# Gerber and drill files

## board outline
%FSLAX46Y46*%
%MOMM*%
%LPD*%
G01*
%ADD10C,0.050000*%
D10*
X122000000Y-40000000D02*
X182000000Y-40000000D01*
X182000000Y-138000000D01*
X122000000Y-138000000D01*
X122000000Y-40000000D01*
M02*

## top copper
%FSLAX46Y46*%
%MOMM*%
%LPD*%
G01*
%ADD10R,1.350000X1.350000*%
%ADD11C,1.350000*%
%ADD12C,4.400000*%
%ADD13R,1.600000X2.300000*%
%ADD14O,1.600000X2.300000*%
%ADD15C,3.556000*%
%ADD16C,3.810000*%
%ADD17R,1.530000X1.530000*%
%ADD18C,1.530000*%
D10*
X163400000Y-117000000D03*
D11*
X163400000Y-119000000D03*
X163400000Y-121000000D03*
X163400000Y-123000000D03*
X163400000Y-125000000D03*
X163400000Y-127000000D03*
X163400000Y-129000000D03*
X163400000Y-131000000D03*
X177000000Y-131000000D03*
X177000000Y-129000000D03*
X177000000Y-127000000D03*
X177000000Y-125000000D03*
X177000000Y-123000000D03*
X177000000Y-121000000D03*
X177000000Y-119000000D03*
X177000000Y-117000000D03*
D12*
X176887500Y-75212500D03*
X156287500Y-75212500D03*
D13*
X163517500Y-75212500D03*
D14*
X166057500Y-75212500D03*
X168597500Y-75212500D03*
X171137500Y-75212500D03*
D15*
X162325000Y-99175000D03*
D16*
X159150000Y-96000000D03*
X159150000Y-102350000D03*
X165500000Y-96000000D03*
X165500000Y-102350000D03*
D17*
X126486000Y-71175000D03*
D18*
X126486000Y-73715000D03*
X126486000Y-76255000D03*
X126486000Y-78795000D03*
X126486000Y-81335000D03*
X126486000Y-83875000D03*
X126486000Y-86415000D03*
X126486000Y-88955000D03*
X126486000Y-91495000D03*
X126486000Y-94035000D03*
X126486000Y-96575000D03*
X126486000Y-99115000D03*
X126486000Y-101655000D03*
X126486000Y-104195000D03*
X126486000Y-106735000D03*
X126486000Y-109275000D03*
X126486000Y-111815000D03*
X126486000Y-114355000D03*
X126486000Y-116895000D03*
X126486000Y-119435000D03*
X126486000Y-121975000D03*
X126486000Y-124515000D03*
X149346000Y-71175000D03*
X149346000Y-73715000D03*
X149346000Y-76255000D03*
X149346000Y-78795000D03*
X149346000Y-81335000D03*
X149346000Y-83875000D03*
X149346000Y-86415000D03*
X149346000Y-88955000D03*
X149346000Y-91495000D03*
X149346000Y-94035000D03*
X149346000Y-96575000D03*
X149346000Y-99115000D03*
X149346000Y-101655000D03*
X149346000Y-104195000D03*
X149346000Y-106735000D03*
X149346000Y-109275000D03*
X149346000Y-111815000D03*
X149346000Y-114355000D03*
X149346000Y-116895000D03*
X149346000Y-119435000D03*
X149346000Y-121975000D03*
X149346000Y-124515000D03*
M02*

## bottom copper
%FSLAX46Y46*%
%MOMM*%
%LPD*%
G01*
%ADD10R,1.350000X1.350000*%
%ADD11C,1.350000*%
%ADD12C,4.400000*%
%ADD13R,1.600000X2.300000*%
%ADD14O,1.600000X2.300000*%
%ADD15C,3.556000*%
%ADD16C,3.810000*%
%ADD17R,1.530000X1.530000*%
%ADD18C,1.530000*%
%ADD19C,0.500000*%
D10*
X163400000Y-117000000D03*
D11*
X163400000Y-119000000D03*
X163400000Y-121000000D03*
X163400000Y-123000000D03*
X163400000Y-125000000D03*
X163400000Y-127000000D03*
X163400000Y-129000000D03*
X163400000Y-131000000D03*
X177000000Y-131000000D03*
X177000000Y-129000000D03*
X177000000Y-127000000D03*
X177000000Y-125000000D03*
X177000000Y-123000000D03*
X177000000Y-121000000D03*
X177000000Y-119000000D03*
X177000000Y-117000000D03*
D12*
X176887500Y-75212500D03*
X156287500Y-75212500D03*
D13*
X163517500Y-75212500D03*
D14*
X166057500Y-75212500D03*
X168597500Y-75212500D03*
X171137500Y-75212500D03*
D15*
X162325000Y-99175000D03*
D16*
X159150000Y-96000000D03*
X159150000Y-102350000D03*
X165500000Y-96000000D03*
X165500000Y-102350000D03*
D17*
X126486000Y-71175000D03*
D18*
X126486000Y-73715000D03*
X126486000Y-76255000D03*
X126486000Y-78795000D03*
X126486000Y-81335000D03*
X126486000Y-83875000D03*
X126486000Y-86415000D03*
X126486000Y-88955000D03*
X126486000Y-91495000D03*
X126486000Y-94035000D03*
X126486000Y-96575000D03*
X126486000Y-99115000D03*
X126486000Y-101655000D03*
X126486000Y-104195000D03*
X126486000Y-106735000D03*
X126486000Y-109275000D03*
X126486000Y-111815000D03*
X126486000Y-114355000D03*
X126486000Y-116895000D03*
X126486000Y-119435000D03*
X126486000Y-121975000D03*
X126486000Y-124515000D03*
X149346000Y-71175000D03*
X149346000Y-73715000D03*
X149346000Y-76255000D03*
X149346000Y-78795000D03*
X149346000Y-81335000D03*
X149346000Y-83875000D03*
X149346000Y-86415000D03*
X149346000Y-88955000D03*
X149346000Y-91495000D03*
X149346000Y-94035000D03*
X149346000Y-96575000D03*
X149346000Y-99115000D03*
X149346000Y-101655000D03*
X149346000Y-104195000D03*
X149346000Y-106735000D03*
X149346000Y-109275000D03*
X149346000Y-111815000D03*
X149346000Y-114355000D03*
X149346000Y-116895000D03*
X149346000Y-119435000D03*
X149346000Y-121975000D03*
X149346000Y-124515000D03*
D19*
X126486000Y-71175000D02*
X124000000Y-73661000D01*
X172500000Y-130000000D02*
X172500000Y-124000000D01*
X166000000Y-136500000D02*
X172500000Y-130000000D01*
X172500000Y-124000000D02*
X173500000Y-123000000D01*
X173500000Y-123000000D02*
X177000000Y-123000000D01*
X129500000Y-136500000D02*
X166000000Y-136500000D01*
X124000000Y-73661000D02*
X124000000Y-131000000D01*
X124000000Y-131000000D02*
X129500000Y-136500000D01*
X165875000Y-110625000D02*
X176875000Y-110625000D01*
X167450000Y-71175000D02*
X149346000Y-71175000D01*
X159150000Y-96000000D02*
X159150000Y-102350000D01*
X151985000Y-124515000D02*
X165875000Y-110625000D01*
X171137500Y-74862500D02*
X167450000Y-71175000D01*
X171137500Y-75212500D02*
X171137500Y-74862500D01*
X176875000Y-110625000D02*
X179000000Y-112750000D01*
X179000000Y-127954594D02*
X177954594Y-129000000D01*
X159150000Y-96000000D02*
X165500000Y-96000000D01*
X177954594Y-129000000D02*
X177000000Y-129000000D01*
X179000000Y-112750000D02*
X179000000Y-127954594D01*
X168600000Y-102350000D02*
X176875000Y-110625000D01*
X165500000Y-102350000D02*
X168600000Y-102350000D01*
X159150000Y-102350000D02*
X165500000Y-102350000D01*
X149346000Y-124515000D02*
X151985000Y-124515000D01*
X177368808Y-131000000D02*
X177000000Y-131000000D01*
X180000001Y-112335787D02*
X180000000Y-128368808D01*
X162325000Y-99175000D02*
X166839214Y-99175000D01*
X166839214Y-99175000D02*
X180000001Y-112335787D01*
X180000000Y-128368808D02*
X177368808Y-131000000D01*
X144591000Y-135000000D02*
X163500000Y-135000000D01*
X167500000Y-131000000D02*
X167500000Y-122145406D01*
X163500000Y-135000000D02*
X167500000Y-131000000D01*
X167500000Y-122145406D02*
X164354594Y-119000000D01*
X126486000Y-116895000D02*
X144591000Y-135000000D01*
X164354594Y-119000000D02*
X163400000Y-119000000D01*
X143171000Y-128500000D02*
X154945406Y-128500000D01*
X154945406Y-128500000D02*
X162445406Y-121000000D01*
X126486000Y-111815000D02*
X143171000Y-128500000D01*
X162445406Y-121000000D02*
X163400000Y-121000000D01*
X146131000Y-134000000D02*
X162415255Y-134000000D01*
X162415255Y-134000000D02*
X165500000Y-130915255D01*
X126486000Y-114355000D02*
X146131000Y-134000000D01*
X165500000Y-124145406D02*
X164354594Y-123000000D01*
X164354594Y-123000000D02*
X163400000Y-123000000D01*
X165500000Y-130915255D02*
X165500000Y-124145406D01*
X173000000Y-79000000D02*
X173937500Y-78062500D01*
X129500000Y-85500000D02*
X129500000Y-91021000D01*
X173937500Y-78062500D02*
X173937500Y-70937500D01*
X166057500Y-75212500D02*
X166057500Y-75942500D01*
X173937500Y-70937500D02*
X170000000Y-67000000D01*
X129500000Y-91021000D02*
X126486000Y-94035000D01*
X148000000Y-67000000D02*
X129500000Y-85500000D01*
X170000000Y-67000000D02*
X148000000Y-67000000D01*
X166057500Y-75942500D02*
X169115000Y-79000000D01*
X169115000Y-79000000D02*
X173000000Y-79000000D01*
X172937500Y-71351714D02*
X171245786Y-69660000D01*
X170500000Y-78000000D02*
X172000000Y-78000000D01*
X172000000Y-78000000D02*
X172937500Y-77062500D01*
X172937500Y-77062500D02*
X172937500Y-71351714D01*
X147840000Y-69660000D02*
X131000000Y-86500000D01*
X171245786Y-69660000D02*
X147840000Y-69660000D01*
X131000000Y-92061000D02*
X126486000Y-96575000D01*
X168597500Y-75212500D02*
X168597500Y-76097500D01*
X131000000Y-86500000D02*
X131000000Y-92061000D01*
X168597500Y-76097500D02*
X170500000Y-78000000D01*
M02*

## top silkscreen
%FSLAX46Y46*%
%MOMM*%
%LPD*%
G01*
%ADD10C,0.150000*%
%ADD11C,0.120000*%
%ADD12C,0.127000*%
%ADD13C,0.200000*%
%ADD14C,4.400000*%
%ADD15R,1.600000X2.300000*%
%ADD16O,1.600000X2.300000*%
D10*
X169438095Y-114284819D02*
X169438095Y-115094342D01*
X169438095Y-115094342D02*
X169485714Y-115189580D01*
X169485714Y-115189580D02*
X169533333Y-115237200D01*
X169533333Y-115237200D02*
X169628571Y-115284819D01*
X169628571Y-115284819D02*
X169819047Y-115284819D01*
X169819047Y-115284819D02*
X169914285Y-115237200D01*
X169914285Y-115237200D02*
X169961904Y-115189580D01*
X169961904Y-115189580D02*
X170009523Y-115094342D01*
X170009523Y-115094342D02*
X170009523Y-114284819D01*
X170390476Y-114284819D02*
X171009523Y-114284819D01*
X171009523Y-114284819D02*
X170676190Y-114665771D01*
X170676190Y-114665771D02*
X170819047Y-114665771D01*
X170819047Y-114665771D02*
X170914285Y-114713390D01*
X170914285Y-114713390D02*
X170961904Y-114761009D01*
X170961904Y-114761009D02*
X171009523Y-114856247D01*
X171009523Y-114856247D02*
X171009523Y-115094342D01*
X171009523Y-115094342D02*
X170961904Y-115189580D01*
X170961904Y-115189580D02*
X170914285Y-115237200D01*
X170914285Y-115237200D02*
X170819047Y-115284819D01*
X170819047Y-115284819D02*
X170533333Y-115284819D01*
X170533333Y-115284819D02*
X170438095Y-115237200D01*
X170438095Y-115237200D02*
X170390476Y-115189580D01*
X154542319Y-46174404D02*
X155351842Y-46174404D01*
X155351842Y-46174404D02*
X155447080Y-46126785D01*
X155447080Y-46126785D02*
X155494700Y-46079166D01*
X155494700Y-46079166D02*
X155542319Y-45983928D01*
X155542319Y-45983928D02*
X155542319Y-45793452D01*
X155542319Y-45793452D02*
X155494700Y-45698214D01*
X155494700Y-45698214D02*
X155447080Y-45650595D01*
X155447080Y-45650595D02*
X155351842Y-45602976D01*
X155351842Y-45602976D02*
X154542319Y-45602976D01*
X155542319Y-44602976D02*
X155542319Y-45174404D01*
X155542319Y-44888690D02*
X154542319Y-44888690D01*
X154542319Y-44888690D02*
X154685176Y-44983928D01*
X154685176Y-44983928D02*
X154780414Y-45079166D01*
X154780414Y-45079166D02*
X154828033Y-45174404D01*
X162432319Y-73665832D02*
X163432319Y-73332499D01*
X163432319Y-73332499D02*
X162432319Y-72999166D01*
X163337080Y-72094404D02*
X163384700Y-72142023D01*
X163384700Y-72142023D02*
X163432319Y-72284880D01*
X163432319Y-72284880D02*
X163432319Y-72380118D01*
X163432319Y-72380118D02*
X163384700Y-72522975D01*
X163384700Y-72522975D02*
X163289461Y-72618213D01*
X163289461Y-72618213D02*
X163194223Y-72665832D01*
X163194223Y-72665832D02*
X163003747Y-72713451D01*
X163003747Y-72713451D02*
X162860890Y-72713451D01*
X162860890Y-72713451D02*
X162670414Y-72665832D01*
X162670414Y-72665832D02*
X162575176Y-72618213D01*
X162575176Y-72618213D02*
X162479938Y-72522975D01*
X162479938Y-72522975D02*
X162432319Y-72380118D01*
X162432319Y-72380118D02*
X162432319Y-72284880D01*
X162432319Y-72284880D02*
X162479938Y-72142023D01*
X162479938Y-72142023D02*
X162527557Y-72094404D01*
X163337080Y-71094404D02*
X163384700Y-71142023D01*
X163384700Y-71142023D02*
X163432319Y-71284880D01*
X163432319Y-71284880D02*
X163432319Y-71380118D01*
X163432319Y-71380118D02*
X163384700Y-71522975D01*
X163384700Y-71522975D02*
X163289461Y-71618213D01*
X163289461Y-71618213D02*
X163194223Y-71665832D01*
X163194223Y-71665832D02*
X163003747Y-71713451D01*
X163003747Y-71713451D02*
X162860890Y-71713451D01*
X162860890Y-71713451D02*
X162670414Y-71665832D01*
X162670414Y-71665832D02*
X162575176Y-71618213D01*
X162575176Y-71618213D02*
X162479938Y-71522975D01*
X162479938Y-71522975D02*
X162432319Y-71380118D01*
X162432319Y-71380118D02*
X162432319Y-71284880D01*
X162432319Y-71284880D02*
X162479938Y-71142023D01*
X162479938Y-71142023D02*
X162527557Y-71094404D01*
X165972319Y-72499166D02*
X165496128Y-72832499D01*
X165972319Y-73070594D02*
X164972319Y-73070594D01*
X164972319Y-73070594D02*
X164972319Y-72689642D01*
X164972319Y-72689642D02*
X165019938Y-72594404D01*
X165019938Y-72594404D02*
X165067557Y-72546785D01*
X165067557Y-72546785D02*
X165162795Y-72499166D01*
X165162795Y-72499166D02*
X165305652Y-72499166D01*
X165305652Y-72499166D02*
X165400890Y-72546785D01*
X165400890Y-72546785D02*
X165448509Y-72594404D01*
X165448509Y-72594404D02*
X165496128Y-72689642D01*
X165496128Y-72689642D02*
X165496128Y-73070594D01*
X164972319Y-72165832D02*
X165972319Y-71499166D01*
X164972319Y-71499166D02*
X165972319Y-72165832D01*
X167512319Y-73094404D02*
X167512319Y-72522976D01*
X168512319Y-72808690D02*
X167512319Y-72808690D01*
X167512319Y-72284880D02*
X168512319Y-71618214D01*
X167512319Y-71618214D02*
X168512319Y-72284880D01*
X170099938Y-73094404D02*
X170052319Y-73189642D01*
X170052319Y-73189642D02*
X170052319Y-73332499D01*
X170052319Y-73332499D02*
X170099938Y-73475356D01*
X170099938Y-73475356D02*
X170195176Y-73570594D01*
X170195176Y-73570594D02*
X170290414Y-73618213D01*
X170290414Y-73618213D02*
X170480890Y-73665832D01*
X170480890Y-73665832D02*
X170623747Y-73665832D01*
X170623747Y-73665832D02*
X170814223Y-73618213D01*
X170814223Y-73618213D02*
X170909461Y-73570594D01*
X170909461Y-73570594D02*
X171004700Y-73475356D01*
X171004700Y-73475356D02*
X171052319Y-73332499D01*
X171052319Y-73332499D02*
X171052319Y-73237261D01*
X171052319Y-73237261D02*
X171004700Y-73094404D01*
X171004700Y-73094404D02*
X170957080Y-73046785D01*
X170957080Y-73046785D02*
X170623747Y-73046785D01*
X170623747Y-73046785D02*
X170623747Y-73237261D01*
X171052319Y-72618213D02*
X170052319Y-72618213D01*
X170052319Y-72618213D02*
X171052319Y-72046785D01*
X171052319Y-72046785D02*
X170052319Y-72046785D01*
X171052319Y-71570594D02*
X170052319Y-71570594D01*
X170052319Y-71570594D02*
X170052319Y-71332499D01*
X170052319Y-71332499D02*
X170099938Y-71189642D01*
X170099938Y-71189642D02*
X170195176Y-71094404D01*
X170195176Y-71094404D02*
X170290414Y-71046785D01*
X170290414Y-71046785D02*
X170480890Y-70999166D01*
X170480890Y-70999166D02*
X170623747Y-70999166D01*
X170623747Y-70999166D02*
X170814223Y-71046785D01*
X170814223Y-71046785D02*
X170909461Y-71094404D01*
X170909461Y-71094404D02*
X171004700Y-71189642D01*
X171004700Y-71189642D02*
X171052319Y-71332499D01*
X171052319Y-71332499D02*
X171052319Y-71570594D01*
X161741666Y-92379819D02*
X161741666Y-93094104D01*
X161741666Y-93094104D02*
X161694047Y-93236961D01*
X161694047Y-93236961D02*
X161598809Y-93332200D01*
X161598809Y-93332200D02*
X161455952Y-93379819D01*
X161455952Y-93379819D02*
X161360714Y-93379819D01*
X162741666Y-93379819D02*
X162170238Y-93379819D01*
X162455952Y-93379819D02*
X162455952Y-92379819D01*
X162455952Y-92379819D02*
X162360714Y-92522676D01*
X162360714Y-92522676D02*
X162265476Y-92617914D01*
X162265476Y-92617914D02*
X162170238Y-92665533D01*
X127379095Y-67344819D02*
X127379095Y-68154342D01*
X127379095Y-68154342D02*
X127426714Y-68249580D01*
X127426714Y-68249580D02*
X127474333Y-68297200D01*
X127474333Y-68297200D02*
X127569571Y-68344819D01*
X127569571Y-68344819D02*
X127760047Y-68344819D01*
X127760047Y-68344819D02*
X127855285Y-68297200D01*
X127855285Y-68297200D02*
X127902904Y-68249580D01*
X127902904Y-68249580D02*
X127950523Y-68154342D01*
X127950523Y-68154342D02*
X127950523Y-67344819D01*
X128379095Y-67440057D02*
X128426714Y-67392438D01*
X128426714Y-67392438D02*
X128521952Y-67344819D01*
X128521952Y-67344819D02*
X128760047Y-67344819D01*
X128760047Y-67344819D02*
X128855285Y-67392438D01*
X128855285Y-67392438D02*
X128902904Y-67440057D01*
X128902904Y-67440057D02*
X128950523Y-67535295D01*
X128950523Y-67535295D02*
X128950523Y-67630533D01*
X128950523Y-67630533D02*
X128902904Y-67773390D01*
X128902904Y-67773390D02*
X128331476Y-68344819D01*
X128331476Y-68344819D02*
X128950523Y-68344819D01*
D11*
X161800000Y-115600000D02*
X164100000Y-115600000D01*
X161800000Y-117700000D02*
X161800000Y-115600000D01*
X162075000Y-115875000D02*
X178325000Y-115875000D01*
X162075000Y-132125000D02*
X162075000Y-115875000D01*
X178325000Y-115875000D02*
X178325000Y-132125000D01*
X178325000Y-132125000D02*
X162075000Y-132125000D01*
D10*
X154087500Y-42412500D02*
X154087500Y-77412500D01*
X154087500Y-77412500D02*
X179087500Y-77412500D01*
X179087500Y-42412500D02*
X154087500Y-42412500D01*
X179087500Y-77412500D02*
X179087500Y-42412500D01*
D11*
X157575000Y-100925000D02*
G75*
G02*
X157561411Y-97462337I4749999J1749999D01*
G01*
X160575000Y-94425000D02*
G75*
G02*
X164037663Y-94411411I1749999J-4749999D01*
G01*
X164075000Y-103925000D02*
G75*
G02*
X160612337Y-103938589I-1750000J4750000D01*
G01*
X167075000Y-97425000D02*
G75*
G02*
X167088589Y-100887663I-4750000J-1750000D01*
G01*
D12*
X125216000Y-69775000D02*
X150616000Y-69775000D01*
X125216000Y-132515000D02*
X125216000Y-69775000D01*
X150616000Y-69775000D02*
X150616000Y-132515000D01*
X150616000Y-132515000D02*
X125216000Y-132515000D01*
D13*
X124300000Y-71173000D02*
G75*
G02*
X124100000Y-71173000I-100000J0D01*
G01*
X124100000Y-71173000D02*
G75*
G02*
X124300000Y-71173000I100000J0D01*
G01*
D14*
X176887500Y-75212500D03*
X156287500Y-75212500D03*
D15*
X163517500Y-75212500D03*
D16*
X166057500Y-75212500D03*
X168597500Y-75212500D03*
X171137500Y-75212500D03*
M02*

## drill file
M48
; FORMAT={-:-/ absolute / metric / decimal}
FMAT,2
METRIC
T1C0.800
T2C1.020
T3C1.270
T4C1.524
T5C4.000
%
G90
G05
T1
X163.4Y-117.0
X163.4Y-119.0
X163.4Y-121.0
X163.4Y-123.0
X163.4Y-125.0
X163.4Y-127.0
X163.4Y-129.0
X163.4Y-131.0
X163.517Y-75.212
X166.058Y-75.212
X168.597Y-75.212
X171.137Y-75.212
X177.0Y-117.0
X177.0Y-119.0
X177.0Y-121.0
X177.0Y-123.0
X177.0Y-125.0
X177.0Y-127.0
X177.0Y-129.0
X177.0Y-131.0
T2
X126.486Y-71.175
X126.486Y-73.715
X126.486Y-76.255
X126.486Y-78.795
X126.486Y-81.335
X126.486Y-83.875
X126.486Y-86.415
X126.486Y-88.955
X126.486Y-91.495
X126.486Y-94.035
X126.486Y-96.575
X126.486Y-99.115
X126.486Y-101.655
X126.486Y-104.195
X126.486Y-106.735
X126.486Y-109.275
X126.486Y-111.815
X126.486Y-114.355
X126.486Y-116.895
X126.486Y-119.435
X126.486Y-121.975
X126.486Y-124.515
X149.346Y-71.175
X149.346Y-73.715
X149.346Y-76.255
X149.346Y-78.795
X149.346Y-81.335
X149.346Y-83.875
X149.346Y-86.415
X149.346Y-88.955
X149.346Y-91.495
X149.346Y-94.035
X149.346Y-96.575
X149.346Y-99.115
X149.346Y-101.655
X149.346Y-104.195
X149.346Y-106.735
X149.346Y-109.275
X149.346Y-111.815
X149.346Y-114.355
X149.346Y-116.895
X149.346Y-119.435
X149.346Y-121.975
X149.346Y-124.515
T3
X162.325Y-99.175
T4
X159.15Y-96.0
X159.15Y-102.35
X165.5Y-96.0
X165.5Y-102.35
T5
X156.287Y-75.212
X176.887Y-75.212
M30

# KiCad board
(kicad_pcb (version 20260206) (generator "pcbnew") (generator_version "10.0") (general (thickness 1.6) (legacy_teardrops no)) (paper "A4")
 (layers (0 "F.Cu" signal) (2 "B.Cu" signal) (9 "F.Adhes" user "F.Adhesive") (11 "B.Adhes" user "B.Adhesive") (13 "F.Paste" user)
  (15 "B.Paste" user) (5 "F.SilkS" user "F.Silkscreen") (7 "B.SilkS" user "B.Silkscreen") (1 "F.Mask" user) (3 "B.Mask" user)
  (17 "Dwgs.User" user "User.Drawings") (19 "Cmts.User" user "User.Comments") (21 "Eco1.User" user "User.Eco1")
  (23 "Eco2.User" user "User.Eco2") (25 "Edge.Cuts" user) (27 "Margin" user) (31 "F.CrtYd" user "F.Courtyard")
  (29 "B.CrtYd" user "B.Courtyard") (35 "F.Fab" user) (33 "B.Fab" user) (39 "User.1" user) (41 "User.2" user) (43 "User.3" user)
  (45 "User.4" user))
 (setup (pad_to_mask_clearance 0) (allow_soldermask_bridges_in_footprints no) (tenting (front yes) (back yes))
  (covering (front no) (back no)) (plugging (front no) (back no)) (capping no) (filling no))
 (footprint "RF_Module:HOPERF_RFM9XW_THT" (layer "F.Cu") (at 163.4 117)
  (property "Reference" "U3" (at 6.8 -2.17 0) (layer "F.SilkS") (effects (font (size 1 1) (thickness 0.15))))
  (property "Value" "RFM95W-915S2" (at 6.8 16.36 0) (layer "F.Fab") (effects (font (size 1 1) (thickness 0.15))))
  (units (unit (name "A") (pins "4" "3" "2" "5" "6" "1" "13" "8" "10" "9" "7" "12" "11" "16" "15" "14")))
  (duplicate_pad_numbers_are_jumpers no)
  (fp_line (start -1.6 -1.4) (end 0.7 -1.4) (stroke (width 0.12) (type solid)) (layer "F.SilkS"))
  (fp_line (start -1.6 0.7) (end -1.6 -1.4) (stroke (width 0.12) (type solid)) (layer "F.SilkS"))
  (fp_line (start -1.325 -1.125) (end 14.925 -1.125) (stroke (width 0.12) (type solid)) (layer "F.SilkS"))
  (fp_line (start -1.325 15.125) (end -1.325 -1.125) (stroke (width 0.12) (type solid)) (layer "F.SilkS"))
  (fp_line (start 14.925 -1.125) (end 14.925 15.125) (stroke (width 0.12) (type solid)) (layer "F.SilkS"))
  (fp_line (start 14.925 15.125) (end -1.325 15.125) (stroke (width 0.12) (type solid)) (layer "F.SilkS"))
  (pad "1" thru_hole rect (at 0 0) (size 1.35 1.35) (drill 0.8) (layers "*.Cu" "*.Mask") (remove_unused_layers no)
   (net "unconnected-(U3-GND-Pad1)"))
  (pad "2" thru_hole circle (at 0 2) (size 1.35 1.35) (drill 0.8) (layers "*.Cu" "*.Mask") (remove_unused_layers no) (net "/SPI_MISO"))
  (pad "3" thru_hole circle (at 0 4) (size 1.35 1.35) (drill 0.8) (layers "*.Cu" "*.Mask") (remove_unused_layers no) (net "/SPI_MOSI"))
  (pad "4" thru_hole circle (at 0 6) (size 1.35 1.35) (drill 0.8) (layers "*.Cu" "*.Mask") (remove_unused_layers no) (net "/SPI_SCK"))
  (pad "5" thru_hole circle (at 0 8) (size 1.35 1.35) (drill 0.8) (layers "*.Cu" "*.Mask") (remove_unused_layers no) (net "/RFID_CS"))
  (pad "6" thru_hole circle (at 0 10) (size 1.35 1.35) (drill 0.8) (layers "*.Cu" "*.Mask") (remove_unused_layers no) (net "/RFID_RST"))
  (pad "7" thru_hole circle (at 0 12) (size 1.35 1.35) (drill 0.8) (layers "*.Cu" "*.Mask") (remove_unused_layers no)
   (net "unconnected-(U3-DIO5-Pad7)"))
  (pad "8" thru_hole circle (at 0 14) (size 1.35 1.35) (drill 0.8) (layers "*.Cu" "*.Mask") (remove_unused_layers no)
   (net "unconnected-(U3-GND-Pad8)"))
  (pad "9" thru_hole circle (at 13.6 14) (size 1.35 1.35) (drill 0.8) (layers "*.Cu" "*.Mask") (remove_unused_layers no) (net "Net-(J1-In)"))
  (pad "10" thru_hole circle (at 13.6 12) (size 1.35 1.35) (drill 0.8) (layers "*.Cu" "*.Mask") (remove_unused_layers no)
   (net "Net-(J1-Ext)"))
  (pad "11" thru_hole circle (at 13.6 10) (size 1.35 1.35) (drill 0.8) (layers "*.Cu" "*.Mask") (remove_unused_layers no)
   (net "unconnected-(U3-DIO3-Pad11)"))
  (pad "12" thru_hole circle (at 13.6 8) (size 1.35 1.35) (drill 0.8) (layers "*.Cu" "*.Mask") (remove_unused_layers no)
   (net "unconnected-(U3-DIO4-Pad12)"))
  (pad "13" thru_hole circle (at 13.6 6) (size 1.35 1.35) (drill 0.8) (layers "*.Cu" "*.Mask") (remove_unused_layers no)
   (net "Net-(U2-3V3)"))
  (pad "14" thru_hole circle (at 13.6 4) (size 1.35 1.35) (drill 0.8) (layers "*.Cu" "*.Mask") (remove_unused_layers no)
   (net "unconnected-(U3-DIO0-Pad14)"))
  (pad "15" thru_hole circle (at 13.6 2) (size 1.35 1.35) (drill 0.8) (layers "*.Cu" "*.Mask") (remove_unused_layers no)
   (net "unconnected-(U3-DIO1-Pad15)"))
  (pad "16" thru_hole circle (at 13.6 0) (size 1.35 1.35) (drill 0.8) (layers "*.Cu" "*.Mask") (remove_unused_layers no)
   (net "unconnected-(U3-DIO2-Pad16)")))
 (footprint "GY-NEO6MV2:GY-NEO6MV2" (layer "F.Cu") (at 154.0875 77.4125 -90)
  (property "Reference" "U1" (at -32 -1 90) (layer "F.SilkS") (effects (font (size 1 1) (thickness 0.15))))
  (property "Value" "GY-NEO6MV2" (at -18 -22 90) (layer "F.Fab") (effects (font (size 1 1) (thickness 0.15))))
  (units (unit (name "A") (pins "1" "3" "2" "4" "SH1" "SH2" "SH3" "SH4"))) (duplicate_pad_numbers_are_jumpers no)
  (fp_line (start -35 0) (end 0 0) (stroke (width 0.15) (type solid)) (layer "F.SilkS"))
  (fp_line (start 0 0) (end 0 -25) (stroke (width 0.15) (type solid)) (layer "F.SilkS"))
  (fp_line (start -35 -25) (end -35 0) (stroke (width 0.15) (type solid)) (layer "F.SilkS"))
  (fp_line (start 0 -25) (end -35 -25) (stroke (width 0.15) (type solid)) (layer "F.SilkS"))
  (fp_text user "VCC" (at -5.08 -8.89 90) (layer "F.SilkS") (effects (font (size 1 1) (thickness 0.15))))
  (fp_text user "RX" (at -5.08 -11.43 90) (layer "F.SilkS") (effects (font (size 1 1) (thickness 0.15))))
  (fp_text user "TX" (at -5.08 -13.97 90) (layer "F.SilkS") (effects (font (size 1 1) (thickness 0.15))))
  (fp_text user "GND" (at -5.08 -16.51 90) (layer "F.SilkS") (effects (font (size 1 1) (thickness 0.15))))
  (pad "" np_thru_hole circle (at -2.2 -22.8 270) (size 4.4 4.4) (drill 4) (layers "*.Cu" "*.Mask" "F.SilkS"))
  (pad "" np_thru_hole circle (at -2.2 -2.2 270) (size 4.4 4.4) (drill 4) (layers "*.Cu" "*.Mask" "F.SilkS"))
  (pad "1" thru_hole rect (at -2.2 -9.43 270) (size 2.3 1.6) (drill 0.8) (layers "*.Cu" "*.Mask" "F.SilkS") (remove_unused_layers no)
   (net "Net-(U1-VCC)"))
  (pad "2" thru_hole oval (at -2.2 -11.97 270) (size 2.3 1.6) (drill 0.8) (layers "*.Cu" "*.Mask" "F.SilkS") (remove_unused_layers no)
   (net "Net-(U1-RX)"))
  (pad "3" thru_hole oval (at -2.2 -14.51 270) (size 2.3 1.6) (drill 0.8) (layers "*.Cu" "*.Mask" "F.SilkS") (remove_unused_layers no)
   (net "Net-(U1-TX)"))
  (pad "4" thru_hole oval (at -2.2 -17.05 270) (size 2.3 1.6) (drill 0.8) (layers "*.Cu" "*.Mask" "F.SilkS") (remove_unused_layers no)
   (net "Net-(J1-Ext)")))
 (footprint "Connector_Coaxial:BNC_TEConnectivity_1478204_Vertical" (layer "F.Cu") (at 162.325 99.175)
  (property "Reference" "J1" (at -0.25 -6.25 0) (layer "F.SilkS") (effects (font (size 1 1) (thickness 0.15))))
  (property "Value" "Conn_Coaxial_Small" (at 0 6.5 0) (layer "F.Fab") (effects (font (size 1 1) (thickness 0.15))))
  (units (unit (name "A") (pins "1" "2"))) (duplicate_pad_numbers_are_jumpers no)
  (fp_arc (start -4.75 1.75) (mid -5.062075 0.019867) (end -4.763589 -1.712663) (stroke (width 0.12) (type solid)) (layer "F.SilkS"))
  (fp_arc (start -1.75 -4.75) (mid -0.019867 -5.062075) (end 1.712663 -4.763589) (stroke (width 0.12) (type solid)) (layer "F.SilkS"))
  (fp_arc (start 1.75 4.75) (mid 0.019867 5.062075) (end -1.712663 4.763589) (stroke (width 0.12) (type solid)) (layer "F.SilkS"))
  (fp_arc (start 4.75 -1.75) (mid 5.062075 -0.019867) (end 4.763589 1.712663) (stroke (width 0.12) (type solid)) (layer "F.SilkS"))
  (pad "1" thru_hole circle (at 0 0) (size 3.556 3.556) (drill 1.27) (layers "*.Cu" "*.Mask") (remove_unused_layers no) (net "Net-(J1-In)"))
  (pad "2" thru_hole circle (at -3.175 -3.175) (size 3.81 3.81) (drill 1.524) (layers "*.Cu" "*.Mask") (remove_unused_layers no)
   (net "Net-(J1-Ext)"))
  (pad "2" thru_hole circle (at -3.175 3.175) (size 3.81 3.81) (drill 1.524) (layers "*.Cu" "*.Mask") (remove_unused_layers no)
   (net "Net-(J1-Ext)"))
  (pad "2" thru_hole circle (at 3.175 -3.175) (size 3.81 3.81) (drill 1.524) (layers "*.Cu" "*.Mask") (remove_unused_layers no)
   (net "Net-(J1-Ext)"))
  (pad "2" thru_hole circle (at 3.175 3.175) (size 3.81 3.81) (drill 1.524) (layers "*.Cu" "*.Mask") (remove_unused_layers no)
   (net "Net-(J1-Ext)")))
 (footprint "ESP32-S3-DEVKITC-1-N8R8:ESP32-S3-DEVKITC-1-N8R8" (layer "F.Cu") (at 137.916 101.145)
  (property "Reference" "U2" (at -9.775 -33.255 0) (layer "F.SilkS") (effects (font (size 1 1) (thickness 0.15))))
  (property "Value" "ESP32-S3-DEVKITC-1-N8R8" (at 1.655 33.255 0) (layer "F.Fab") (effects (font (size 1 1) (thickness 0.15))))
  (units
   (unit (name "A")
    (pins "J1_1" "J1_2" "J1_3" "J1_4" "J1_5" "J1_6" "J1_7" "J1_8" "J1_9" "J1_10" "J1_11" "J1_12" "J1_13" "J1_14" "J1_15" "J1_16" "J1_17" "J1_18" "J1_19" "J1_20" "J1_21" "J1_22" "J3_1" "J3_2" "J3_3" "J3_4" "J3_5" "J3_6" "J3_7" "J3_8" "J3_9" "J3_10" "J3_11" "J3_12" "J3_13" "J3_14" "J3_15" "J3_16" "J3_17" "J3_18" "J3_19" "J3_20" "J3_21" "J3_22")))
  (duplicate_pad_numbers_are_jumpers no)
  (fp_line (start -12.7 -31.37) (end 12.7 -31.37) (stroke (width 0.127) (type solid)) (layer "F.SilkS"))
  (fp_line (start -12.7 31.37) (end -12.7 -31.37) (stroke (width 0.127) (type solid)) (layer "F.SilkS"))
  (fp_line (start 12.7 -31.37) (end 12.7 31.37) (stroke (width 0.127) (type solid)) (layer "F.SilkS"))
  (fp_line (start 12.7 31.37) (end -12.7 31.37) (stroke (width 0.127) (type solid)) (layer "F.SilkS"))
  (fp_circle (center -13.716 -29.972) (end -13.616 -29.972) (stroke (width 0.2) (type solid)) (fill no) (layer "F.SilkS"))
  (pad "J1_1" thru_hole rect (at -11.43 -29.97) (size 1.53 1.53) (drill 1.02) (layers "*.Cu" "*.Mask") (remove_unused_layers no)
   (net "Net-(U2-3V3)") (solder_mask_margin 0.102))
  (pad "J1_2" thru_hole circle (at -11.43 -27.43) (size 1.53 1.53) (drill 1.02) (layers "*.Cu" "*.Mask") (remove_unused_layers no)
   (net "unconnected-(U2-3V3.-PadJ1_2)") (solder_mask_margin 0.102))
  (pad "J1_3" thru_hole circle (at -11.43 -24.89) (size 1.53 1.53) (drill 1.02) (layers "*.Cu" "*.Mask") (remove_unused_layers no)
   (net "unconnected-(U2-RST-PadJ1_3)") (solder_mask_margin 0.102))
  (pad "J1_4" thru_hole circle (at -11.43 -22.35) (size 1.53 1.53) (drill 1.02) (layers "*.Cu" "*.Mask") (remove_unused_layers no)
   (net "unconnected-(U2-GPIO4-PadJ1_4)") (solder_mask_margin 0.102))
  (pad "J1_5" thru_hole circle (at -11.43 -19.81) (size 1.53 1.53) (drill 1.02) (layers "*.Cu" "*.Mask") (remove_unused_layers no)
   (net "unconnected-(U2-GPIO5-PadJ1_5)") (solder_mask_margin 0.102))
  (pad "J1_6" thru_hole circle (at -11.43 -17.27) (size 1.53 1.53) (drill 1.02) (layers "*.Cu" "*.Mask") (remove_unused_layers no)
   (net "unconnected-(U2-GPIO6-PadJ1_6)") (solder_mask_margin 0.102))
  (pad "J1_7" thru_hole circle (at -11.43 -14.73) (size 1.53 1.53) (drill 1.02) (layers "*.Cu" "*.Mask") (remove_unused_layers no)
   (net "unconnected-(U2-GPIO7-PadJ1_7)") (solder_mask_margin 0.102))
  (pad "J1_8" thru_hole circle (at -11.43 -12.19) (size 1.53 1.53) (drill 1.02) (layers "*.Cu" "*.Mask") (remove_unused_layers no)
   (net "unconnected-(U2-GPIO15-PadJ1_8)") (solder_mask_margin 0.102))
  (pad "J1_9" thru_hole circle (at -11.43 -9.65) (size 1.53 1.53) (drill 1.02) (layers "*.Cu" "*.Mask") (remove_unused_layers no)
   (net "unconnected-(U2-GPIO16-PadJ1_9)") (solder_mask_margin 0.102))
  (pad "J1_10" thru_hole circle (at -11.43 -7.11) (size 1.53 1.53) (drill 1.02) (layers "*.Cu" "*.Mask") (remove_unused_layers no)
   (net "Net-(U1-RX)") (solder_mask_margin 0.102))
  (pad "J1_11" thru_hole circle (at -11.43 -4.57) (size 1.53 1.53) (drill 1.02) (layers "*.Cu" "*.Mask") (remove_unused_layers no)
   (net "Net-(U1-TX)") (solder_mask_margin 0.102))
  (pad "J1_12" thru_hole circle (at -11.43 -2.03) (size 1.53 1.53) (drill 1.02) (layers "*.Cu" "*.Mask") (remove_unused_layers no)
   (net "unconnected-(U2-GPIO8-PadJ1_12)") (solder_mask_margin 0.102))
  (pad "J1_13" thru_hole circle (at -11.43 0.51) (size 1.53 1.53) (drill 1.02) (layers "*.Cu" "*.Mask") (remove_unused_layers no)
   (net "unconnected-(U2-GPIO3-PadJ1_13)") (solder_mask_margin 0.102))
  (pad "J1_14" thru_hole circle (at -11.43 3.05) (size 1.53 1.53) (drill 1.02) (layers "*.Cu" "*.Mask") (remove_unused_layers no)
   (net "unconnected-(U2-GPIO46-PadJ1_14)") (solder_mask_margin 0.102))
  (pad "J1_15" thru_hole circle (at -11.43 5.59) (size 1.53 1.53) (drill 1.02) (layers "*.Cu" "*.Mask") (remove_unused_layers no)
   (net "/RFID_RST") (solder_mask_margin 0.102))
  (pad "J1_16" thru_hole circle (at -11.43 8.13) (size 1.53 1.53) (drill 1.02) (layers "*.Cu" "*.Mask") (remove_unused_layers no)
   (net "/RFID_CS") (solder_mask_margin 0.102))
  (pad "J1_17" thru_hole circle (at -11.43 10.67) (size 1.53 1.53) (drill 1.02) (layers "*.Cu" "*.Mask") (remove_unused_layers no)
   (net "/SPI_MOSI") (solder_mask_margin 0.102))
  (pad "J1_18" thru_hole circle (at -11.43 13.21) (size 1.53 1.53) (drill 1.02) (layers "*.Cu" "*.Mask") (remove_unused_layers no)
   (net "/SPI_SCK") (solder_mask_margin 0.102))
  (pad "J1_19" thru_hole circle (at -11.43 15.75) (size 1.53 1.53) (drill 1.02) (layers "*.Cu" "*.Mask") (remove_unused_layers no)
   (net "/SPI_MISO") (solder_mask_margin 0.102))
  (pad "J1_20" thru_hole circle (at -11.43 18.29) (size 1.53 1.53) (drill 1.02) (layers "*.Cu" "*.Mask") (remove_unused_layers no)
   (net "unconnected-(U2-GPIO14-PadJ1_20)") (solder_mask_margin 0.102))
  (pad "J1_21" thru_hole circle (at -11.43 20.83) (size 1.53 1.53) (drill 1.02) (layers "*.Cu" "*.Mask") (remove_unused_layers no)
   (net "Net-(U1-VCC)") (solder_mask_margin 0.102))
  (pad "J1_22" thru_hole circle (at -11.43 23.37) (size 1.53 1.53) (drill 1.02) (layers "*.Cu" "*.Mask") (remove_unused_layers no)
   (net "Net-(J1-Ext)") (solder_mask_margin 0.102))
  (pad "J3_1" thru_hole circle (at 11.43 -29.97) (size 1.53 1.53) (drill 1.02) (layers "*.Cu" "*.Mask") (remove_unused_layers no)
   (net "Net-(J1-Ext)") (solder_mask_margin 0.102))
  (pad "J3_2" thru_hole circle (at 11.43 -27.43) (size 1.53 1.53) (drill 1.02) (layers "*.Cu" "*.Mask") (remove_unused_layers no)
   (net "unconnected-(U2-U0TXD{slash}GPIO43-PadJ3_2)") (solder_mask_margin 0.102))
  (pad "J3_3" thru_hole circle (at 11.43 -24.89) (size 1.53 1.53) (drill 1.02) (layers "*.Cu" "*.Mask") (remove_unused_layers no)
   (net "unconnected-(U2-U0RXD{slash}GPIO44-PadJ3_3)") (solder_mask_margin 0.102))
  (pad "J3_4" thru_hole circle (at 11.43 -22.35) (size 1.53 1.53) (drill 1.02) (layers "*.Cu" "*.Mask") (remove_unused_layers no)
   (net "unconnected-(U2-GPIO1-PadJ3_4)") (solder_mask_margin 0.102))
  (pad "J3_5" thru_hole circle (at 11.43 -19.81) (size 1.53 1.53) (drill 1.02) (layers "*.Cu" "*.Mask") (remove_unused_layers no)
   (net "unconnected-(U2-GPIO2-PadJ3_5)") (solder_mask_margin 0.102))
  (pad "J3_6" thru_hole circle (at 11.43 -17.27) (size 1.53 1.53) (drill 1.02) (layers "*.Cu" "*.Mask") (remove_unused_layers no)
   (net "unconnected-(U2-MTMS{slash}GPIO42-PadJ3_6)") (solder_mask_margin 0.102))
  (pad "J3_7" thru_hole circle (at 11.43 -14.73) (size 1.53 1.53) (drill 1.02) (layers "*.Cu" "*.Mask") (remove_unused_layers no)
   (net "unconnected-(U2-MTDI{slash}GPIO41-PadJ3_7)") (solder_mask_margin 0.102))
  (pad "J3_8" thru_hole circle (at 11.43 -12.19) (size 1.53 1.53) (drill 1.02) (layers "*.Cu" "*.Mask") (remove_unused_layers no)
   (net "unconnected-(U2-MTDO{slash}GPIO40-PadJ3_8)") (solder_mask_margin 0.102))
  (pad "J3_9" thru_hole circle (at 11.43 -9.65) (size 1.53 1.53) (drill 1.02) (layers "*.Cu" "*.Mask") (remove_unused_layers no)
   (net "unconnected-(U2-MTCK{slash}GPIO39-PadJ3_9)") (solder_mask_margin 0.102))
  (pad "J3_10" thru_hole circle (at 11.43 -7.11) (size 1.53 1.53) (drill 1.02) (layers "*.Cu" "*.Mask") (remove_unused_layers no)
   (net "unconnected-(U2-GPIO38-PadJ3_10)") (solder_mask_margin 0.102))
  (pad "J3_11" thru_hole circle (at 11.43 -4.57) (size 1.53 1.53) (drill 1.02) (layers "*.Cu" "*.Mask") (remove_unused_layers no)
   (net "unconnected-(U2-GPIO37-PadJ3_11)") (solder_mask_margin 0.102))
  (pad "J3_12" thru_hole circle (at 11.43 -2.03) (size 1.53 1.53) (drill 1.02) (layers "*.Cu" "*.Mask") (remove_unused_layers no)
   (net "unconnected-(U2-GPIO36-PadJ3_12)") (solder_mask_margin 0.102))
  (pad "J3_13" thru_hole circle (at 11.43 0.51) (size 1.53 1.53) (drill 1.02) (layers "*.Cu" "*.Mask") (remove_unused_layers no)
   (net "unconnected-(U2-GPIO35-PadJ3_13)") (solder_mask_margin 0.102))
  (pad "J3_14" thru_hole circle (at 11.43 3.05) (size 1.53 1.53) (drill 1.02) (layers "*.Cu" "*.Mask") (remove_unused_layers no)
   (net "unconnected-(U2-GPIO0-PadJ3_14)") (solder_mask_margin 0.102))
  (pad "J3_15" thru_hole circle (at 11.43 5.59) (size 1.53 1.53) (drill 1.02) (layers "*.Cu" "*.Mask") (remove_unused_layers no)
   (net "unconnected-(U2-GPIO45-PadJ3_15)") (solder_mask_margin 0.102))
  (pad "J3_16" thru_hole circle (at 11.43 8.13) (size 1.53 1.53) (drill 1.02) (layers "*.Cu" "*.Mask") (remove_unused_layers no)
   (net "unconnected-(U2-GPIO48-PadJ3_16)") (solder_mask_margin 0.102))
  (pad "J3_17" thru_hole circle (at 11.43 10.67) (size 1.53 1.53) (drill 1.02) (layers "*.Cu" "*.Mask") (remove_unused_layers no)
   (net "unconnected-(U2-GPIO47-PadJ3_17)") (solder_mask_margin 0.102))
  (pad "J3_18" thru_hole circle (at 11.43 13.21) (size 1.53 1.53) (drill 1.02) (layers "*.Cu" "*.Mask") (remove_unused_layers no)
   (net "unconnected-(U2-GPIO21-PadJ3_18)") (solder_mask_margin 0.102))
  (pad "J3_19" thru_hole circle (at 11.43 15.75) (size 1.53 1.53) (drill 1.02) (layers "*.Cu" "*.Mask") (remove_unused_layers no)
   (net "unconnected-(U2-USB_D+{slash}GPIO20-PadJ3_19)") (solder_mask_margin 0.102))
  (pad "J3_20" thru_hole circle (at 11.43 18.29) (size 1.53 1.53) (drill 1.02) (layers "*.Cu" "*.Mask") (remove_unused_layers no)
   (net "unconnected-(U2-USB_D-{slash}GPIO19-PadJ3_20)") (solder_mask_margin 0.102))
  (pad "J3_21" thru_hole circle (at 11.43 20.83) (size 1.53 1.53) (drill 1.02) (layers "*.Cu" "*.Mask") (remove_unused_layers no)
   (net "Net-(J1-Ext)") (solder_mask_margin 0.102))
  (pad "J3_22" thru_hole circle (at 11.43 23.37) (size 1.53 1.53) (drill 1.02) (layers "*.Cu" "*.Mask") (remove_unused_layers no)
   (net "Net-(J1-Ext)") (solder_mask_margin 0.102)))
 (gr_rect (start 122 40) (end 182 138) (stroke (width 0.05) (type solid)) (fill no) (layer "Edge.Cuts"))
 (segment (start 126.486 71.175) (end 124 73.661) (width 0.5) (layer "B.Cu") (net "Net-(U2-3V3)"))
 (segment (start 172.5 130) (end 172.5 124) (width 0.5) (layer "B.Cu") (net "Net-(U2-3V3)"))
 (segment (start 166 136.5) (end 172.5 130) (width 0.5) (layer "B.Cu") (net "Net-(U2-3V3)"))
 (segment (start 172.5 124) (end 173.5 123) (width 0.5) (layer "B.Cu") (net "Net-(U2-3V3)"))
 (segment (start 173.5 123) (end 177 123) (width 0.5) (layer "B.Cu") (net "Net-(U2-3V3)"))
 (segment (start 129.5 136.5) (end 166 136.5) (width 0.5) (layer "B.Cu") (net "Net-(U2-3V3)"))
 (segment (start 124 73.661) (end 124 131) (width 0.5) (layer "B.Cu") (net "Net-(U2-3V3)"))
 (segment (start 124 131) (end 129.5 136.5) (width 0.5) (layer "B.Cu") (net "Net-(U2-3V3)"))
 (segment (start 165.875 110.625) (end 176.875 110.625) (width 0.5) (layer "B.Cu") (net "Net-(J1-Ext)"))
 (segment (start 167.45 71.175) (end 149.346 71.175) (width 0.5) (layer "B.Cu") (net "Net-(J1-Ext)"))
 (segment (start 159.15 96) (end 159.15 102.35) (width 0.5) (layer "B.Cu") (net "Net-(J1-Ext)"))
 (segment (start 151.985 124.515) (end 165.875 110.625) (width 0.5) (layer "B.Cu") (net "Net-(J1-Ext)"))
 (segment (start 171.1375 74.8625) (end 167.45 71.175) (width 0.5) (layer "B.Cu") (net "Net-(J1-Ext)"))
 (segment (start 171.1375 75.2125) (end 171.1375 74.8625) (width 0.5) (layer "B.Cu") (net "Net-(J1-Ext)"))
 (segment (start 176.875 110.625) (end 179 112.75) (width 0.5) (layer "B.Cu") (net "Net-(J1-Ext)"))
 (segment (start 179 127.954594) (end 177.954594 129) (width 0.5) (layer "B.Cu") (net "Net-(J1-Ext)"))
 (segment (start 159.15 96) (end 165.5 96) (width 0.5) (layer "B.Cu") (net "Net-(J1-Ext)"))
 (segment (start 177.954594 129) (end 177 129) (width 0.5) (layer "B.Cu") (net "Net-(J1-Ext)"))
 (segment (start 179 112.75) (end 179 127.954594) (width 0.5) (layer "B.Cu") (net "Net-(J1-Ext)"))
 (segment (start 168.6 102.35) (end 176.875 110.625) (width 0.5) (layer "B.Cu") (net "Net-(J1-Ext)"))
 (segment (start 165.5 102.35) (end 168.6 102.35) (width 0.5) (layer "B.Cu") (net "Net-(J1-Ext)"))
 (segment (start 159.15 102.35) (end 165.5 102.35) (width 0.5) (layer "B.Cu") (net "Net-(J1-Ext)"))
 (segment (start 149.346 124.515) (end 151.985 124.515) (width 0.5) (layer "B.Cu") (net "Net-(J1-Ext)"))
 (segment (start 177.368808 131) (end 177 131) (width 0.5) (layer "B.Cu") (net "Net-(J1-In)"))
 (segment (start 180.000001 112.335787) (end 180 128.368808) (width 0.5) (layer "B.Cu") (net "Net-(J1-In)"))
 (segment (start 162.325 99.175) (end 166.839214 99.175) (width 0.5) (layer "B.Cu") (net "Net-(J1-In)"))
 (segment (start 166.839214 99.175) (end 180.000001 112.335787) (width 0.5) (layer "B.Cu") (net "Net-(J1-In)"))
 (segment (start 180 128.368808) (end 177.368808 131) (width 0.5) (layer "B.Cu") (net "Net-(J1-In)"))
 (segment (start 144.591 135) (end 163.5 135) (width 0.5) (layer "B.Cu") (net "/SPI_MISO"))
 (segment (start 167.5 131) (end 167.5 122.145406) (width 0.5) (layer "B.Cu") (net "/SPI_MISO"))
 (segment (start 163.5 135) (end 167.5 131) (width 0.5) (layer "B.Cu") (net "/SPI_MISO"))
 (segment (start 167.5 122.145406) (end 164.354594 119) (width 0.5) (layer "B.Cu") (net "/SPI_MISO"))
 (segment (start 126.486 116.895) (end 144.591 135) (width 0.5) (layer "B.Cu") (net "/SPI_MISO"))
 (segment (start 164.354594 119) (end 163.4 119) (width 0.5) (layer "B.Cu") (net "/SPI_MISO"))
 (segment (start 143.171 128.5) (end 154.945406 128.5) (width 0.5) (layer "B.Cu") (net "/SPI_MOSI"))
 (segment (start 154.945406 128.5) (end 162.445406 121) (width 0.5) (layer "B.Cu") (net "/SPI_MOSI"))
 (segment (start 126.486 111.815) (end 143.171 128.5) (width 0.5) (layer "B.Cu") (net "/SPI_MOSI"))
 (segment (start 162.445406 121) (end 163.4 121) (width 0.5) (layer "B.Cu") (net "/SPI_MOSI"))
 (segment (start 146.131 134) (end 162.415255 134) (width 0.5) (layer "B.Cu") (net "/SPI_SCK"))
 (segment (start 162.415255 134) (end 165.5 130.915255) (width 0.5) (layer "B.Cu") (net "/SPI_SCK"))
 (segment (start 126.486 114.355) (end 146.131 134) (width 0.5) (layer "B.Cu") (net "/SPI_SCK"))
 (segment (start 165.5 124.145406) (end 164.354594 123) (width 0.5) (layer "B.Cu") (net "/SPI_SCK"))
 (segment (start 164.354594 123) (end 163.4 123) (width 0.5) (layer "B.Cu") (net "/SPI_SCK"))
 (segment (start 165.5 130.915255) (end 165.5 124.145406) (width 0.5) (layer "B.Cu") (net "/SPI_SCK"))
 (segment (start 173 79) (end 173.9375 78.0625) (width 0.5) (layer "B.Cu") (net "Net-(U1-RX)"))
 (segment (start 129.5 85.5) (end 129.5 91.021) (width 0.5) (layer "B.Cu") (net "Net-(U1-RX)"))
 (segment (start 173.9375 78.0625) (end 173.9375 70.9375) (width 0.5) (layer "B.Cu") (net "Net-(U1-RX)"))
 (segment (start 166.0575 75.2125) (end 166.0575 75.9425) (width 0.5) (layer "B.Cu") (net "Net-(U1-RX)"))
 (segment (start 173.9375 70.9375) (end 170 67) (width 0.5) (layer "B.Cu") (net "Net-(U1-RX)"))
 (segment (start 129.5 91.021) (end 126.486 94.035) (width 0.5) (layer "B.Cu") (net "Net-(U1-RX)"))
 (segment (start 148 67) (end 129.5 85.5) (width 0.5) (layer "B.Cu") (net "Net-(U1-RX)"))
 (segment (start 170 67) (end 148 67) (width 0.5) (layer "B.Cu") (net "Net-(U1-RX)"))
 (segment (start 166.0575 75.9425) (end 169.115 79) (width 0.5) (layer "B.Cu") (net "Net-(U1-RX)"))
 (segment (start 169.115 79) (end 173 79) (width 0.5) (layer "B.Cu") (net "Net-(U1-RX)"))
 (segment (start 172.9375 71.351714) (end 171.245786 69.66) (width 0.5) (layer "B.Cu") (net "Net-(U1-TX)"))
 (segment (start 170.5 78) (end 172 78) (width 0.5) (layer "B.Cu") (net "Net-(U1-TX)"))
 (segment (start 172 78) (end 172.9375 77.0625) (width 0.5) (layer "B.Cu") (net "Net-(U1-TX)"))
 (segment (start 172.9375 77.0625) (end 172.9375 71.351714) (width 0.5) (layer "B.Cu") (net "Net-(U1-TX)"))
 (segment (start 147.84 69.66) (end 131 86.5) (width 0.5) (layer "B.Cu") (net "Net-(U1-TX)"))
 (segment (start 171.245786 69.66) (end 147.84 69.66) (width 0.5) (layer "B.Cu") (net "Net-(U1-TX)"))
 (segment (start 131 92.061) (end 126.486 96.575) (width 0.5) (layer "B.Cu") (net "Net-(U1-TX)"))
 (segment (start 168.5975 75.2125) (end 168.5975 76.0975) (width 0.5) (layer "B.Cu") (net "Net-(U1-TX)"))
 (segment (start 131 86.5) (end 131 92.061) (width 0.5) (layer "B.Cu") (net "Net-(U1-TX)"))
 (segment (start 168.5975 76.0975) (end 170.5 78) (width 0.5) (layer "B.Cu") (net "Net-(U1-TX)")))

